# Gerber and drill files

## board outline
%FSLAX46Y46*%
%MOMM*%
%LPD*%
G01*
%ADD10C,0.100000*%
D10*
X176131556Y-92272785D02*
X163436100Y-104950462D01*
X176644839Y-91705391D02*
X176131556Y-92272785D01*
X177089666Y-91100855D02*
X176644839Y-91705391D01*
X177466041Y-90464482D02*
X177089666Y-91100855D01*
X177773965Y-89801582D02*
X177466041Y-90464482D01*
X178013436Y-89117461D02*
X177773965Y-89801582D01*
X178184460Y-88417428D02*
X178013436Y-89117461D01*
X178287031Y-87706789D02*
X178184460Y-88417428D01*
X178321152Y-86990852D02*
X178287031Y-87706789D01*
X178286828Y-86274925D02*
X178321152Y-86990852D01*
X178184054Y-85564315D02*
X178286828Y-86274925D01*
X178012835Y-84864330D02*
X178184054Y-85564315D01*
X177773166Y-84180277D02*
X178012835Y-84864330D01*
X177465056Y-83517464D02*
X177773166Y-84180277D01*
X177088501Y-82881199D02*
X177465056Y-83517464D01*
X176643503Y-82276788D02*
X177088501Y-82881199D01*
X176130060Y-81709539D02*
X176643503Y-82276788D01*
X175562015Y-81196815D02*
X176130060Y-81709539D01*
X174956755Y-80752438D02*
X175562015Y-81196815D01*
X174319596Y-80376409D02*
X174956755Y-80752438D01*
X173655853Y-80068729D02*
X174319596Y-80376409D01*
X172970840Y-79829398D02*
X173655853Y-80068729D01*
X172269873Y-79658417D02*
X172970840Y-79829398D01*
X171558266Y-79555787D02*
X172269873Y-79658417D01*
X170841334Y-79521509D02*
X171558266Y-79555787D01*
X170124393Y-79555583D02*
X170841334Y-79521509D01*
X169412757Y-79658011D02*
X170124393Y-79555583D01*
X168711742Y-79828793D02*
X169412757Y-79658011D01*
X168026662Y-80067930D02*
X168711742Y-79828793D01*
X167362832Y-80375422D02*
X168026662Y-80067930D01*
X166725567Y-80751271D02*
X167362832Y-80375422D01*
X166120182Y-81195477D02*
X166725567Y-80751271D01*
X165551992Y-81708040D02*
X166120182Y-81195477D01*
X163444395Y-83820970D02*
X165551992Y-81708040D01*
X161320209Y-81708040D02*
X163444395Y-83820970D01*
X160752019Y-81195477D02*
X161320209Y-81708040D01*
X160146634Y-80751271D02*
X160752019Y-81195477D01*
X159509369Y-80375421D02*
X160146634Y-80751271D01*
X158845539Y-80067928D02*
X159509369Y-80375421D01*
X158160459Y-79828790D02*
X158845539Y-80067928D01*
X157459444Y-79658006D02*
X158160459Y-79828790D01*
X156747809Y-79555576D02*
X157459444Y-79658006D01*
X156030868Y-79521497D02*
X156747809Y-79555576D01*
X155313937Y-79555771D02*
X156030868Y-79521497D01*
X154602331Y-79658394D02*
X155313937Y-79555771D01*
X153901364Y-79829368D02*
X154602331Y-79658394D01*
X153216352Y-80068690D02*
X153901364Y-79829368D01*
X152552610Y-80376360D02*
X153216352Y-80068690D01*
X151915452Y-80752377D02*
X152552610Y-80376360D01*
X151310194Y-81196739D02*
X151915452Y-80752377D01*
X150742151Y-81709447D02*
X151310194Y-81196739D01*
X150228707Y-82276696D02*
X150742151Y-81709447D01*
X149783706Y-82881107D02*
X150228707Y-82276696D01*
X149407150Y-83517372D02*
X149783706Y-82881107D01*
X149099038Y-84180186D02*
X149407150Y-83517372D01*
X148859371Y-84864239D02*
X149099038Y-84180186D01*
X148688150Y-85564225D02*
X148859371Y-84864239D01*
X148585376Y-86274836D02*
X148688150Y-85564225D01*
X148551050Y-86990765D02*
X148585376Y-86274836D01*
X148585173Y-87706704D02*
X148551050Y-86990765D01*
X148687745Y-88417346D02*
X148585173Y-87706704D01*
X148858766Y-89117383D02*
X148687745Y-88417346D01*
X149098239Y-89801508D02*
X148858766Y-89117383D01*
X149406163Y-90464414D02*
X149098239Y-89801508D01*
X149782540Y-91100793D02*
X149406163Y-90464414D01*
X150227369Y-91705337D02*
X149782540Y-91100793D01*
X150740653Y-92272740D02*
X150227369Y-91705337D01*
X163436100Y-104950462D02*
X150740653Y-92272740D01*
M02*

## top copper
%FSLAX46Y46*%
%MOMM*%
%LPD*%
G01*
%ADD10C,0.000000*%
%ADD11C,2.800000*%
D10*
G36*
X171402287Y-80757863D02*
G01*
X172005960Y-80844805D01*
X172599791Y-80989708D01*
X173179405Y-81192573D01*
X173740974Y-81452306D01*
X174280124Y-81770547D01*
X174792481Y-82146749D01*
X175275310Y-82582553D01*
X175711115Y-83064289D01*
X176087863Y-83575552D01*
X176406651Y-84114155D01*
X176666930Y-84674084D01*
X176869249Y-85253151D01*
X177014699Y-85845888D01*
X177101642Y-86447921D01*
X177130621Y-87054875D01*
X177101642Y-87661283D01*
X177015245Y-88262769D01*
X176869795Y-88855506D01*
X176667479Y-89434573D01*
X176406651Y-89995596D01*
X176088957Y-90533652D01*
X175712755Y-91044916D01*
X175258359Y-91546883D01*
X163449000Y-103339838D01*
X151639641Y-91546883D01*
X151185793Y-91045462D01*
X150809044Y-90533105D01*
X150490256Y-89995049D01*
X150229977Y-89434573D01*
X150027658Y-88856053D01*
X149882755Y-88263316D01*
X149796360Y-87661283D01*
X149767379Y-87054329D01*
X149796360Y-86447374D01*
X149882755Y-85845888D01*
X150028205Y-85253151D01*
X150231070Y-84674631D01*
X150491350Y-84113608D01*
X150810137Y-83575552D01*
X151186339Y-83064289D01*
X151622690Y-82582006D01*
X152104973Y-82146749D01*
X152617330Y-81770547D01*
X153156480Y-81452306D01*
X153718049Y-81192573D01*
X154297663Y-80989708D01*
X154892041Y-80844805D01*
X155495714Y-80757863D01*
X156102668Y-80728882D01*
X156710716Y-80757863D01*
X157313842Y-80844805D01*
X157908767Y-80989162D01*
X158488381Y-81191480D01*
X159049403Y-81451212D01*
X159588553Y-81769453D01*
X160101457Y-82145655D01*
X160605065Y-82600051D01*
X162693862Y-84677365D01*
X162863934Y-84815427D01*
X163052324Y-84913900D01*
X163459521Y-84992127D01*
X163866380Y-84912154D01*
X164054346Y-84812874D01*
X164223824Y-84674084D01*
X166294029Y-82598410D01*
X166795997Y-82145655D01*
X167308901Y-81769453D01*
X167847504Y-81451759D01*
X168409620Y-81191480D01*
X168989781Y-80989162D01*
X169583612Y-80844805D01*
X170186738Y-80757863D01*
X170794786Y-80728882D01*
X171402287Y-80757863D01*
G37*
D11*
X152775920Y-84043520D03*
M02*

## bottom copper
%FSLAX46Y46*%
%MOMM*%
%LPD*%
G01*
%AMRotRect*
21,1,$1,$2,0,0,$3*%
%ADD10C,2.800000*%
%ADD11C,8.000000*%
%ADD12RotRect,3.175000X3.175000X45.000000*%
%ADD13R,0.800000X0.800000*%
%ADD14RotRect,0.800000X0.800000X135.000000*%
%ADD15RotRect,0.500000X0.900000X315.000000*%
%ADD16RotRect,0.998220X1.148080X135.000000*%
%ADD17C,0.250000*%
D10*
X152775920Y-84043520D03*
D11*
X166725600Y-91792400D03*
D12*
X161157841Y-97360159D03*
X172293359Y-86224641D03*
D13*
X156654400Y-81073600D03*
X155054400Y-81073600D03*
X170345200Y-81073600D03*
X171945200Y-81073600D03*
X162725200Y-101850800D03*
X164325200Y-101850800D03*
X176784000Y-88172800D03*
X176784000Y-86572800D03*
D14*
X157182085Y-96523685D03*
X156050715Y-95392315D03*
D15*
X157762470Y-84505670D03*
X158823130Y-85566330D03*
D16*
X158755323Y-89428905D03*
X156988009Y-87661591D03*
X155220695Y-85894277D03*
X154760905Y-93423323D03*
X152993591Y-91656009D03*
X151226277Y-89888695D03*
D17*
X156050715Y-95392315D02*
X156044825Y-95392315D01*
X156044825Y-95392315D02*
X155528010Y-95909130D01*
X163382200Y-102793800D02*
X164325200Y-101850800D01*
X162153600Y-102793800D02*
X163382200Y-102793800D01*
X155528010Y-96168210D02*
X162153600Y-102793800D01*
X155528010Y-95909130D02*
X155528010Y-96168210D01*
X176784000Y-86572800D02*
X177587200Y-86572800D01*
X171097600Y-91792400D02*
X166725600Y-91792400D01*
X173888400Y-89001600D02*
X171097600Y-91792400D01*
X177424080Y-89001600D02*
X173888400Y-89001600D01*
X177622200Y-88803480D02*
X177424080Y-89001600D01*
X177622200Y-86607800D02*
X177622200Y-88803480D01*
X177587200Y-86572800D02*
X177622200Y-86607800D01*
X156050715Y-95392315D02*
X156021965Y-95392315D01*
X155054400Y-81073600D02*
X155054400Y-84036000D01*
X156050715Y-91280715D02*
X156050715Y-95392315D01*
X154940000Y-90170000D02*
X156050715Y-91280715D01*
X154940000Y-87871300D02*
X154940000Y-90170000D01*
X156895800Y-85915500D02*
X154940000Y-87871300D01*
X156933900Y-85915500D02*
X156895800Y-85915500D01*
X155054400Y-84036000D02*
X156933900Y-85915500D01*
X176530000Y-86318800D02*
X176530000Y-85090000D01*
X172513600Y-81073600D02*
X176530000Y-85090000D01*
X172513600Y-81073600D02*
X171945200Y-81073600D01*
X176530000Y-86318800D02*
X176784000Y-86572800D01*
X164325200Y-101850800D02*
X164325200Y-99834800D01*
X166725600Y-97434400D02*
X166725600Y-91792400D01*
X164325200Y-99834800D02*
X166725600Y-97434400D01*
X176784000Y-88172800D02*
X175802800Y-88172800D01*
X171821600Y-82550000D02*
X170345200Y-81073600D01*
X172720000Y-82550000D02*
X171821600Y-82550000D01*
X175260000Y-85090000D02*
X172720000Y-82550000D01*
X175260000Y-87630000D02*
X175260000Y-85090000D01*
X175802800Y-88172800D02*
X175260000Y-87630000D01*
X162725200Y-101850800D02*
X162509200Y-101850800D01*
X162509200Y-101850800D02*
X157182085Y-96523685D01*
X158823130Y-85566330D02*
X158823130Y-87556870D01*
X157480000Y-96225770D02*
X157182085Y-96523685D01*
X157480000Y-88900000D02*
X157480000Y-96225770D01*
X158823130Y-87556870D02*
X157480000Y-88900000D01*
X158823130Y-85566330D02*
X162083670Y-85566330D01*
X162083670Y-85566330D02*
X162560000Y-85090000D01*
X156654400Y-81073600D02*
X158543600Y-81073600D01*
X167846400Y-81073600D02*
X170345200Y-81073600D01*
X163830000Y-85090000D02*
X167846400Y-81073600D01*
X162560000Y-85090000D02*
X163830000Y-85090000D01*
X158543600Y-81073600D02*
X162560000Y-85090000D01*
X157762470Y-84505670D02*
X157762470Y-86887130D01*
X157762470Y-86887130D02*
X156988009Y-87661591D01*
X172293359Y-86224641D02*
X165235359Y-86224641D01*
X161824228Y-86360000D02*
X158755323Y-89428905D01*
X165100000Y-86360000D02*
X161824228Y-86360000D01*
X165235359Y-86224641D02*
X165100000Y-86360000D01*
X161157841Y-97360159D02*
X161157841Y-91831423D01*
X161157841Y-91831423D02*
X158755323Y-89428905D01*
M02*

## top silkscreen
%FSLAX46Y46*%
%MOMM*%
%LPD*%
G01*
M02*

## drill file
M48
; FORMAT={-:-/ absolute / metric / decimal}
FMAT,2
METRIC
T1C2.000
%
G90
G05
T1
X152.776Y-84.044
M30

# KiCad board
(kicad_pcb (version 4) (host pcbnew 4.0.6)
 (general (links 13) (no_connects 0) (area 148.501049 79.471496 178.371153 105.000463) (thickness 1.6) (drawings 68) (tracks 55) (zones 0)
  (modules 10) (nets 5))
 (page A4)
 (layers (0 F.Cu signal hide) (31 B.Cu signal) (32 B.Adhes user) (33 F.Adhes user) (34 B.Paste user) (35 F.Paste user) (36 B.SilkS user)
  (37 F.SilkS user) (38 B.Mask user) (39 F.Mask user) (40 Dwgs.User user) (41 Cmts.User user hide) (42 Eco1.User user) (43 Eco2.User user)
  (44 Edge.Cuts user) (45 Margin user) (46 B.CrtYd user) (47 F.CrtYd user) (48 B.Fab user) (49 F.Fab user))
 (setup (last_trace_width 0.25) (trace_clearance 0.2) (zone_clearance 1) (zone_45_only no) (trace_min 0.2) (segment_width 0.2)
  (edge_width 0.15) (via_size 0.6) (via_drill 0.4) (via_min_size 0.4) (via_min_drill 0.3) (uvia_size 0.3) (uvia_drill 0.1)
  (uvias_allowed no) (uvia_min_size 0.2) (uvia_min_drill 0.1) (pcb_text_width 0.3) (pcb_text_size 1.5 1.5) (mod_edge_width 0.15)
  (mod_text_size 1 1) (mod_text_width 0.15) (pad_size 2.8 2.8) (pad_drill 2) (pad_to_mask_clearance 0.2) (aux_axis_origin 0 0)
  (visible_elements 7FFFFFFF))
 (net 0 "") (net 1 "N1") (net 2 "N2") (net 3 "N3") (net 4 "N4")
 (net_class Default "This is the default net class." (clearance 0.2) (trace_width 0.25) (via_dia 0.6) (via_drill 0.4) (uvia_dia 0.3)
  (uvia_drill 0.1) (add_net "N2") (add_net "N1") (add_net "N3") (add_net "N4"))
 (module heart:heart (layer F.Cu) (at 163.449 92.03436)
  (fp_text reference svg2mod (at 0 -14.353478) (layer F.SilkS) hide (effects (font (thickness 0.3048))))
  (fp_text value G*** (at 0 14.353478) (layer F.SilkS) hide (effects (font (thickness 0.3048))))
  (fp_poly
   (pts (xy -7.346332 -11.305478) (xy -7.953286 -11.276497) (xy -8.556959 -11.189555) (xy -9.151337 -11.044652) (xy -9.730951 -10.841787)
    (xy -10.29252 -10.582054) (xy -10.83167 -10.263813) (xy -11.344027 -9.887611) (xy -11.82631 -9.452354) (xy -12.262661 -8.970071)
    (xy -12.638863 -8.458808) (xy -12.95765 -7.920752) (xy -13.21793 -7.359729) (xy -13.420795 -6.781209) (xy -13.566245 -6.188472)
    (xy -13.65264 -5.586986) (xy -13.681621 -4.980031) (xy -13.65264 -4.373077) (xy -13.566245 -3.771044) (xy -13.421342 -3.178307)
    (xy -13.219023 -2.599787) (xy -12.958744 -2.039311) (xy -12.639956 -1.501255) (xy -12.263207 -0.988898) (xy -11.809359 -0.487477)
    (xy 0 11.305478) (xy 11.809359 -0.487477) (xy 12.263755 -0.989444) (xy 12.639957 -1.500708) (xy 12.957651 -2.038764)
    (xy 13.218479 -2.599787) (xy 13.420795 -3.178854) (xy 13.566245 -3.771591) (xy 13.652642 -4.373077) (xy 13.681621 -4.979485)
    (xy 13.652642 -5.586439) (xy 13.565699 -6.188472) (xy 13.420249 -6.781209) (xy 13.21793 -7.360276) (xy 12.957651 -7.920205)
    (xy 12.638863 -8.458808) (xy 12.262115 -8.970071) (xy 11.82631 -9.451807) (xy 11.343481 -9.887611) (xy 10.831124 -10.263813)
    (xy 10.291974 -10.582054) (xy 9.730405 -10.841787) (xy 9.150791 -11.044652) (xy 8.55696 -11.189555) (xy 7.953287 -11.276497)
    (xy 7.345786 -11.305478) (xy 6.737738 -11.276497) (xy 6.134612 -11.189555) (xy 5.540781 -11.045198) (xy 4.96062 -10.84288)
    (xy 4.398504 -10.582601) (xy 3.859901 -10.264907) (xy 3.346997 -9.888705) (xy 2.845029 -9.43595) (xy 0.774824 -7.360276)
    (xy 0.605346 -7.221486) (xy 0.41738 -7.122206) (xy 0.010521 -7.042233) (xy -0.396676 -7.12046) (xy -0.585066 -7.218933)
    (xy -0.755138 -7.356995) (xy -2.843935 -9.434309) (xy -3.347543 -9.888705) (xy -3.860447 -10.264907) (xy -4.399597 -10.583148)
    (xy -4.960619 -10.84288) (xy -5.540233 -11.045198) (xy -6.135158 -11.189555) (xy -6.738284 -11.276497) (xy -7.346332 -11.305478))
   (layer F.Cu) (width 0)))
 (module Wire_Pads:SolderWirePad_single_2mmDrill (layer F.Cu) (at 152.77592 84.04352)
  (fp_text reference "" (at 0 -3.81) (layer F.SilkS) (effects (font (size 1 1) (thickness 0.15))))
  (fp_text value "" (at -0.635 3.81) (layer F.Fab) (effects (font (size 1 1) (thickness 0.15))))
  (pad 1 thru_hole circle (at 0 0) (size 2.8 2.8) (drill 2) (layers *.Cu *.Mask)))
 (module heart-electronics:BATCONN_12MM (layer B.Cu) (at 166.7256 91.7924 45)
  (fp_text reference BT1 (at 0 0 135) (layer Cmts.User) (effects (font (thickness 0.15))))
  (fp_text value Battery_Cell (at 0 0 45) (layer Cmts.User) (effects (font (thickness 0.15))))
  (pad 2 smd circle (at 0 0 45) (size 8 8) (layers B.Cu B.Paste B.Mask) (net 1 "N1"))
  (pad 1 smd rect (at -7.874 0 45) (size 3.175 3.175) (layers B.Cu B.Paste B.Mask) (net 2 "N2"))
  (pad 1 smd rect (at 7.874 0 45) (size 3.175 3.175) (layers B.Cu B.Paste B.Mask) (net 2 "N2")))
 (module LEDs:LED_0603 (layer B.Cu) (at 155.8544 81.0736)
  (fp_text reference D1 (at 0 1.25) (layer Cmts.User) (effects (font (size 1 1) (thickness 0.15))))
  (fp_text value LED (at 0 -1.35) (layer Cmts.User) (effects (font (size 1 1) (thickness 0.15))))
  (pad 2 smd rect (at 0.8 0 180) (size 0.8 0.8) (layers B.Cu B.Paste B.Mask) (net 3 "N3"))
  (pad 1 smd rect (at -0.8 0 180) (size 0.8 0.8) (layers B.Cu B.Paste B.Mask) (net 1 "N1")))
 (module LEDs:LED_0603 (layer B.Cu) (at 171.1452 81.0736 180)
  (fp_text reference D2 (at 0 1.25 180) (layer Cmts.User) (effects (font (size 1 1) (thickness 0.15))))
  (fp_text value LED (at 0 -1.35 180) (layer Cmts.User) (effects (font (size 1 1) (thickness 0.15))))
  (pad 2 smd rect (at 0.8 0) (size 0.8 0.8) (layers B.Cu B.Paste B.Mask) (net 3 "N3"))
  (pad 1 smd rect (at -0.8 0) (size 0.8 0.8) (layers B.Cu B.Paste B.Mask) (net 1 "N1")))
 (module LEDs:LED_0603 (layer B.Cu) (at 163.5252 101.8508 180)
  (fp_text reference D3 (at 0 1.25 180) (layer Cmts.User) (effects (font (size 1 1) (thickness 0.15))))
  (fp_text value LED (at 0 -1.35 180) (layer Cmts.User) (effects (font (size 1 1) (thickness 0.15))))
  (pad 2 smd rect (at 0.8 0) (size 0.8 0.8) (layers B.Cu B.Paste B.Mask) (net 3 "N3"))
  (pad 1 smd rect (at -0.8 0) (size 0.8 0.8) (layers B.Cu B.Paste B.Mask) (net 1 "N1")))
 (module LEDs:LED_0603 (layer B.Cu) (at 176.784 87.3728 270)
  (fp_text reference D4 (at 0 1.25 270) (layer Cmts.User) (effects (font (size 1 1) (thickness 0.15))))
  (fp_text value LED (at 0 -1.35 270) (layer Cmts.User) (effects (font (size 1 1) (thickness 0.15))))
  (pad 2 smd rect (at 0.8 0 90) (size 0.8 0.8) (layers B.Cu B.Paste B.Mask) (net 3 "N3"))
  (pad 1 smd rect (at -0.8 0 90) (size 0.8 0.8) (layers B.Cu B.Paste B.Mask) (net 1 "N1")))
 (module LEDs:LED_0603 (layer B.Cu) (at 156.6164 95.958 315)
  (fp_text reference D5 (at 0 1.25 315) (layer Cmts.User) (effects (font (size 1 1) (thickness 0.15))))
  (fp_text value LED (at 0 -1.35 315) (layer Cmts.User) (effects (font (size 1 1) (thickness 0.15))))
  (pad 2 smd rect (at 0.8 0 135) (size 0.8 0.8) (layers B.Cu B.Paste B.Mask) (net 3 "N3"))
  (pad 1 smd rect (at -0.8 0 135) (size 0.8 0.8) (layers B.Cu B.Paste B.Mask) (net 1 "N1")))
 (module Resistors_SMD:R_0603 (layer B.Cu) (at 158.2928 85.036 315)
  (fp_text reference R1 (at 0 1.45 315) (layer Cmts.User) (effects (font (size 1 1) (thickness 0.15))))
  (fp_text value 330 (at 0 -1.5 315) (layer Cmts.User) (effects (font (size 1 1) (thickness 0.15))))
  (pad 1 smd rect (at -0.75 0 315) (size 0.5 0.9) (layers B.Cu B.Paste B.Mask) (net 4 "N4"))
  (pad 2 smd rect (at 0.75 0 315) (size 0.5 0.9) (layers B.Cu B.Paste B.Mask) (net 3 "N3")))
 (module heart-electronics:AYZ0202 (layer B.Cu) (at 154.9908 89.6588 135)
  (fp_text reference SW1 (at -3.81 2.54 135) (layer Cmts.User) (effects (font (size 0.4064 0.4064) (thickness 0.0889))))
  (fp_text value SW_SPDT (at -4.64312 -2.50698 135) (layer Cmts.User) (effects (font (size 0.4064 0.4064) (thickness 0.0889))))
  (pad 1 smd rect (at -2.49936 2.82448 135) (size 0.99822 1.14808) (layers B.Cu B.Paste B.Mask) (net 2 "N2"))
  (pad 2 smd rect (at 0 2.82448 135) (size 0.99822 1.14808) (layers B.Cu B.Paste B.Mask) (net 4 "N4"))
  (pad 3 smd rect (at 2.49936 2.82448 135) (size 0.99822 1.14808) (layers B.Cu B.Paste B.Mask))
  (pad 4 smd rect (at -2.49936 -2.82448 135) (size 0.99822 1.14808) (layers B.Cu B.Paste B.Mask))
  (pad 5 smd rect (at 0 -2.82448 135) (size 0.99822 1.14808) (layers B.Cu B.Paste B.Mask))
  (pad 6 smd rect (at 2.49936 -2.82448 135) (size 0.99822 1.14808) (layers B.Cu B.Paste B.Mask)))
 (gr_line (start 176.131556 92.272785) (end 163.4361 104.950462) (layer Edge.Cuts) (width 0.1))
 (gr_line (start 176.644839 91.705391) (end 176.131556 92.272785) (layer Edge.Cuts) (width 0.1))
 (gr_line (start 177.089666 91.100855) (end 176.644839 91.705391) (layer Edge.Cuts) (width 0.1))
 (gr_line (start 177.466041 90.464482) (end 177.089666 91.100855) (layer Edge.Cuts) (width 0.1))
 (gr_line (start 177.773965 89.801582) (end 177.466041 90.464482) (layer Edge.Cuts) (width 0.1))
 (gr_line (start 178.013436 89.117461) (end 177.773965 89.801582) (layer Edge.Cuts) (width 0.1))
 (gr_line (start 178.18446 88.417428) (end 178.013436 89.117461) (layer Edge.Cuts) (width 0.1))
 (gr_line (start 178.287031 87.706789) (end 178.18446 88.417428) (layer Edge.Cuts) (width 0.1))
 (gr_line (start 178.321152 86.990852) (end 178.287031 87.706789) (layer Edge.Cuts) (width 0.1))
 (gr_line (start 178.286828 86.274925) (end 178.321152 86.990852) (layer Edge.Cuts) (width 0.1))
 (gr_line (start 178.184054 85.564315) (end 178.286828 86.274925) (layer Edge.Cuts) (width 0.1))
 (gr_line (start 178.012835 84.86433) (end 178.184054 85.564315) (layer Edge.Cuts) (width 0.1))
 (gr_line (start 177.773166 84.180277) (end 178.012835 84.86433) (layer Edge.Cuts) (width 0.1))
 (gr_line (start 177.465056 83.517464) (end 177.773166 84.180277) (layer Edge.Cuts) (width 0.1))
 (gr_line (start 177.088501 82.881199) (end 177.465056 83.517464) (layer Edge.Cuts) (width 0.1))
 (gr_line (start 176.643503 82.276788) (end 177.088501 82.881199) (layer Edge.Cuts) (width 0.1))
 (gr_line (start 176.13006 81.709539) (end 176.643503 82.276788) (layer Edge.Cuts) (width 0.1))
 (gr_line (start 175.562015 81.196815) (end 176.13006 81.709539) (layer Edge.Cuts) (width 0.1))
 (gr_line (start 174.956755 80.752438) (end 175.562015 81.196815) (layer Edge.Cuts) (width 0.1))
 (gr_line (start 174.319596 80.376409) (end 174.956755 80.752438) (layer Edge.Cuts) (width 0.1))
 (gr_line (start 173.655853 80.068729) (end 174.319596 80.376409) (layer Edge.Cuts) (width 0.1))
 (gr_line (start 172.97084 79.829398) (end 173.655853 80.068729) (layer Edge.Cuts) (width 0.1))
 (gr_line (start 172.269873 79.658417) (end 172.97084 79.829398) (layer Edge.Cuts) (width 0.1))
 (gr_line (start 171.558266 79.555787) (end 172.269873 79.658417) (layer Edge.Cuts) (width 0.1))
 (gr_line (start 170.841334 79.521509) (end 171.558266 79.555787) (layer Edge.Cuts) (width 0.1))
 (gr_line (start 170.124393 79.555583) (end 170.841334 79.521509) (layer Edge.Cuts) (width 0.1))
 (gr_line (start 169.412757 79.658011) (end 170.124393 79.555583) (layer Edge.Cuts) (width 0.1))
 (gr_line (start 168.711742 79.828793) (end 169.412757 79.658011) (layer Edge.Cuts) (width 0.1))
 (gr_line (start 168.026662 80.06793) (end 168.711742 79.828793) (layer Edge.Cuts) (width 0.1))
 (gr_line (start 167.362832 80.375422) (end 168.026662 80.06793) (layer Edge.Cuts) (width 0.1))
 (gr_line (start 166.725567 80.751271) (end 167.362832 80.375422) (layer Edge.Cuts) (width 0.1))
 (gr_line (start 166.120182 81.195477) (end 166.725567 80.751271) (layer Edge.Cuts) (width 0.1))
 (gr_line (start 165.551992 81.70804) (end 166.120182 81.195477) (layer Edge.Cuts) (width 0.1))
 (gr_line (start 163.444395 83.82097) (end 165.551992 81.70804) (layer Edge.Cuts) (width 0.1))
 (gr_line (start 161.320209 81.70804) (end 163.444395 83.82097) (layer Edge.Cuts) (width 0.1))
 (gr_line (start 160.752019 81.195477) (end 161.320209 81.70804) (layer Edge.Cuts) (width 0.1))
 (gr_line (start 160.146634 80.751271) (end 160.752019 81.195477) (layer Edge.Cuts) (width 0.1))
 (gr_line (start 159.509369 80.375421) (end 160.146634 80.751271) (layer Edge.Cuts) (width 0.1))
 (gr_line (start 158.845539 80.067928) (end 159.509369 80.375421) (layer Edge.Cuts) (width 0.1))
 (gr_line (start 158.160459 79.82879) (end 158.845539 80.067928) (layer Edge.Cuts) (width 0.1))
 (gr_line (start 157.459444 79.658006) (end 158.160459 79.82879) (layer Edge.Cuts) (width 0.1))
 (gr_line (start 156.747809 79.555576) (end 157.459444 79.658006) (layer Edge.Cuts) (width 0.1))
 (gr_line (start 156.030868 79.521497) (end 156.747809 79.555576) (layer Edge.Cuts) (width 0.1))
 (gr_line (start 155.313937 79.555771) (end 156.030868 79.521497) (layer Edge.Cuts) (width 0.1))
 (gr_line (start 154.602331 79.658394) (end 155.313937 79.555771) (layer Edge.Cuts) (width 0.1))
 (gr_line (start 153.901364 79.829368) (end 154.602331 79.658394) (layer Edge.Cuts) (width 0.1))
 (gr_line (start 153.216352 80.06869) (end 153.901364 79.829368) (layer Edge.Cuts) (width 0.1))
 (gr_line (start 152.55261 80.37636) (end 153.216352 80.06869) (layer Edge.Cuts) (width 0.1))
 (gr_line (start 151.915452 80.752377) (end 152.55261 80.37636) (layer Edge.Cuts) (width 0.1))
 (gr_line (start 151.310194 81.196739) (end 151.915452 80.752377) (layer Edge.Cuts) (width 0.1))
 (gr_line (start 150.742151 81.709447) (end 151.310194 81.196739) (layer Edge.Cuts) (width 0.1))
 (gr_line (start 150.228707 82.276696) (end 150.742151 81.709447) (layer Edge.Cuts) (width 0.1))
 (gr_line (start 149.783706 82.881107) (end 150.228707 82.276696) (layer Edge.Cuts) (width 0.1))
 (gr_line (start 149.40715 83.517372) (end 149.783706 82.881107) (layer Edge.Cuts) (width 0.1))
 (gr_line (start 149.099038 84.180186) (end 149.40715 83.517372) (layer Edge.Cuts) (width 0.1))
 (gr_line (start 148.859371 84.864239) (end 149.099038 84.180186) (layer Edge.Cuts) (width 0.1))
 (gr_line (start 148.68815 85.564225) (end 148.859371 84.864239) (layer Edge.Cuts) (width 0.1))
 (gr_line (start 148.585376 86.274836) (end 148.68815 85.564225) (layer Edge.Cuts) (width 0.1))
 (gr_line (start 148.55105 86.990765) (end 148.585376 86.274836) (layer Edge.Cuts) (width 0.1))
 (gr_line (start 148.585173 87.706704) (end 148.55105 86.990765) (layer Edge.Cuts) (width 0.1))
 (gr_line (start 148.687745 88.417346) (end 148.585173 87.706704) (layer Edge.Cuts) (width 0.1))
 (gr_line (start 148.858766 89.117383) (end 148.687745 88.417346) (layer Edge.Cuts) (width 0.1))
 (gr_line (start 149.098239 89.801508) (end 148.858766 89.117383) (layer Edge.Cuts) (width 0.1))
 (gr_line (start 149.406163 90.464414) (end 149.098239 89.801508) (layer Edge.Cuts) (width 0.1))
 (gr_line (start 149.78254 91.100793) (end 149.406163 90.464414) (layer Edge.Cuts) (width 0.1))
 (gr_line (start 150.227369 91.705337) (end 149.78254 91.100793) (layer Edge.Cuts) (width 0.1))
 (gr_line (start 150.740653 92.27274) (end 150.227369 91.705337) (layer Edge.Cuts) (width 0.1))
 (gr_line (start 163.4361 104.950462) (end 150.740653 92.27274) (layer Edge.Cuts) (width 0.1))
 (segment (start 156.050715 95.392315) (end 156.044825 95.392315) (width 0.25) (layer B.Cu) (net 1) (status C00000))
 (segment (start 156.044825 95.392315) (end 155.52801 95.90913) (width 0.25) (layer B.Cu) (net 1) (status 400000))
 (segment (start 163.3822 102.7938) (end 164.3252 101.8508) (width 0.25) (layer B.Cu) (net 1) (status 800000))
 (segment (start 162.1536 102.7938) (end 163.3822 102.7938) (width 0.25) (layer B.Cu) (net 1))
 (segment (start 155.52801 96.16821) (end 162.1536 102.7938) (width 0.25) (layer B.Cu) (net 1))
 (segment (start 155.52801 95.90913) (end 155.52801 96.16821) (width 0.25) (layer B.Cu) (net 1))
 (segment (start 176.784 86.5728) (end 177.5872 86.5728) (width 0.25) (layer B.Cu) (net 1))
 (segment (start 171.0976 91.7924) (end 166.7256 91.7924) (width 0.25) (layer B.Cu) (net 1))
 (segment (start 173.8884 89.0016) (end 171.0976 91.7924) (width 0.25) (layer B.Cu) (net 1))
 (segment (start 177.42408 89.0016) (end 173.8884 89.0016) (width 0.25) (layer B.Cu) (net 1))
 (segment (start 177.6222 88.80348) (end 177.42408 89.0016) (width 0.25) (layer B.Cu) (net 1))
 (segment (start 177.6222 86.6078) (end 177.6222 88.80348) (width 0.25) (layer B.Cu) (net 1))
 (segment (start 177.5872 86.5728) (end 177.6222 86.6078) (width 0.25) (layer B.Cu) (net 1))
 (segment (start 156.050715 95.392315) (end 156.021965 95.392315) (width 0.25) (layer B.Cu) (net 1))
 (segment (start 155.0544 81.0736) (end 155.0544 84.036) (width 0.25) (layer B.Cu) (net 1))
 (segment (start 156.050715 91.280715) (end 156.050715 95.392315) (width 0.25) (layer B.Cu) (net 1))
 (segment (start 154.94 90.17) (end 156.050715 91.280715) (width 0.25) (layer B.Cu) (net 1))
 (segment (start 154.94 87.8713) (end 154.94 90.17) (width 0.25) (layer B.Cu) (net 1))
 (segment (start 156.8958 85.9155) (end 154.94 87.8713) (width 0.25) (layer B.Cu) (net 1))
 (segment (start 156.9339 85.9155) (end 156.8958 85.9155) (width 0.25) (layer B.Cu) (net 1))
 (segment (start 155.0544 84.036) (end 156.9339 85.9155) (width 0.25) (layer B.Cu) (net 1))
 (segment (start 176.53 86.3188) (end 176.53 85.09) (width 0.25) (layer B.Cu) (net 1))
 (segment (start 172.5136 81.0736) (end 176.53 85.09) (width 0.25) (layer B.Cu) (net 1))
 (segment (start 172.5136 81.0736) (end 171.9452 81.0736) (width 0.25) (layer B.Cu) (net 1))
 (segment (start 176.53 86.3188) (end 176.784 86.5728) (width 0.25) (layer B.Cu) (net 1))
 (segment (start 164.3252 101.8508) (end 164.3252 99.8348) (width 0.25) (layer B.Cu) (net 1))
 (segment (start 166.7256 97.4344) (end 166.7256 91.7924) (width 0.25) (layer B.Cu) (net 1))
 (segment (start 164.3252 99.8348) (end 166.7256 97.4344) (width 0.25) (layer B.Cu) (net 1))
 (segment (start 176.784 88.1728) (end 175.8028 88.1728) (width 0.25) (layer B.Cu) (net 3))
 (segment (start 171.8216 82.55) (end 170.3452 81.0736) (width 0.25) (layer B.Cu) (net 3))
 (segment (start 172.72 82.55) (end 171.8216 82.55) (width 0.25) (layer B.Cu) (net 3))
 (segment (start 175.26 85.09) (end 172.72 82.55) (width 0.25) (layer B.Cu) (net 3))
 (segment (start 175.26 87.63) (end 175.26 85.09) (width 0.25) (layer B.Cu) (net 3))
 (segment (start 175.8028 88.1728) (end 175.26 87.63) (width 0.25) (layer B.Cu) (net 3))
 (segment (start 162.7252 101.8508) (end 162.5092 101.8508) (width 0.25) (layer B.Cu) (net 3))
 (segment (start 162.5092 101.8508) (end 157.182085 96.523685) (width 0.25) (layer B.Cu) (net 3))
 (segment (start 158.82313 85.56633) (end 158.82313 87.55687) (width 0.25) (layer B.Cu) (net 3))
 (segment (start 157.48 96.22577) (end 157.182085 96.523685) (width 0.25) (layer B.Cu) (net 3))
 (segment (start 157.48 88.9) (end 157.48 96.22577) (width 0.25) (layer B.Cu) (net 3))
 (segment (start 158.82313 87.55687) (end 157.48 88.9) (width 0.25) (layer B.Cu) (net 3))
 (segment (start 158.82313 85.56633) (end 162.08367 85.56633) (width 0.25) (layer B.Cu) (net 3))
 (segment (start 162.08367 85.56633) (end 162.56 85.09) (width 0.25) (layer B.Cu) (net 3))
 (segment (start 156.6544 81.0736) (end 158.5436 81.0736) (width 0.25) (layer B.Cu) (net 3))
 (segment (start 167.8464 81.0736) (end 170.3452 81.0736) (width 0.25) (layer B.Cu) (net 3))
 (segment (start 163.83 85.09) (end 167.8464 81.0736) (width 0.25) (layer B.Cu) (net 3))
 (segment (start 162.56 85.09) (end 163.83 85.09) (width 0.25) (layer B.Cu) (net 3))
 (segment (start 158.5436 81.0736) (end 162.56 85.09) (width 0.25) (layer B.Cu) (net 3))
 (segment (start 157.76247 84.50567) (end 157.76247 86.88713) (width 0.25) (layer B.Cu) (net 4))
 (segment (start 157.76247 86.88713) (end 156.988009 87.661591) (width 0.25) (layer B.Cu) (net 4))
 (segment (start 172.293359 86.224641) (end 165.235359 86.224641) (width 0.25) (layer B.Cu) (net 2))
 (segment (start 161.824228 86.36) (end 158.755323 89.428905) (width 0.25) (layer B.Cu) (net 2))
 (segment (start 165.1 86.36) (end 161.824228 86.36) (width 0.25) (layer B.Cu) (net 2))
 (segment (start 165.235359 86.224641) (end 165.1 86.36) (width 0.25) (layer B.Cu) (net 2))
 (segment (start 161.157841 97.360159) (end 161.157841 91.831423) (width 0.25) (layer B.Cu) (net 2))
 (segment (start 161.157841 91.831423) (end 158.755323 89.428905) (width 0.25) (layer B.Cu) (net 2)))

